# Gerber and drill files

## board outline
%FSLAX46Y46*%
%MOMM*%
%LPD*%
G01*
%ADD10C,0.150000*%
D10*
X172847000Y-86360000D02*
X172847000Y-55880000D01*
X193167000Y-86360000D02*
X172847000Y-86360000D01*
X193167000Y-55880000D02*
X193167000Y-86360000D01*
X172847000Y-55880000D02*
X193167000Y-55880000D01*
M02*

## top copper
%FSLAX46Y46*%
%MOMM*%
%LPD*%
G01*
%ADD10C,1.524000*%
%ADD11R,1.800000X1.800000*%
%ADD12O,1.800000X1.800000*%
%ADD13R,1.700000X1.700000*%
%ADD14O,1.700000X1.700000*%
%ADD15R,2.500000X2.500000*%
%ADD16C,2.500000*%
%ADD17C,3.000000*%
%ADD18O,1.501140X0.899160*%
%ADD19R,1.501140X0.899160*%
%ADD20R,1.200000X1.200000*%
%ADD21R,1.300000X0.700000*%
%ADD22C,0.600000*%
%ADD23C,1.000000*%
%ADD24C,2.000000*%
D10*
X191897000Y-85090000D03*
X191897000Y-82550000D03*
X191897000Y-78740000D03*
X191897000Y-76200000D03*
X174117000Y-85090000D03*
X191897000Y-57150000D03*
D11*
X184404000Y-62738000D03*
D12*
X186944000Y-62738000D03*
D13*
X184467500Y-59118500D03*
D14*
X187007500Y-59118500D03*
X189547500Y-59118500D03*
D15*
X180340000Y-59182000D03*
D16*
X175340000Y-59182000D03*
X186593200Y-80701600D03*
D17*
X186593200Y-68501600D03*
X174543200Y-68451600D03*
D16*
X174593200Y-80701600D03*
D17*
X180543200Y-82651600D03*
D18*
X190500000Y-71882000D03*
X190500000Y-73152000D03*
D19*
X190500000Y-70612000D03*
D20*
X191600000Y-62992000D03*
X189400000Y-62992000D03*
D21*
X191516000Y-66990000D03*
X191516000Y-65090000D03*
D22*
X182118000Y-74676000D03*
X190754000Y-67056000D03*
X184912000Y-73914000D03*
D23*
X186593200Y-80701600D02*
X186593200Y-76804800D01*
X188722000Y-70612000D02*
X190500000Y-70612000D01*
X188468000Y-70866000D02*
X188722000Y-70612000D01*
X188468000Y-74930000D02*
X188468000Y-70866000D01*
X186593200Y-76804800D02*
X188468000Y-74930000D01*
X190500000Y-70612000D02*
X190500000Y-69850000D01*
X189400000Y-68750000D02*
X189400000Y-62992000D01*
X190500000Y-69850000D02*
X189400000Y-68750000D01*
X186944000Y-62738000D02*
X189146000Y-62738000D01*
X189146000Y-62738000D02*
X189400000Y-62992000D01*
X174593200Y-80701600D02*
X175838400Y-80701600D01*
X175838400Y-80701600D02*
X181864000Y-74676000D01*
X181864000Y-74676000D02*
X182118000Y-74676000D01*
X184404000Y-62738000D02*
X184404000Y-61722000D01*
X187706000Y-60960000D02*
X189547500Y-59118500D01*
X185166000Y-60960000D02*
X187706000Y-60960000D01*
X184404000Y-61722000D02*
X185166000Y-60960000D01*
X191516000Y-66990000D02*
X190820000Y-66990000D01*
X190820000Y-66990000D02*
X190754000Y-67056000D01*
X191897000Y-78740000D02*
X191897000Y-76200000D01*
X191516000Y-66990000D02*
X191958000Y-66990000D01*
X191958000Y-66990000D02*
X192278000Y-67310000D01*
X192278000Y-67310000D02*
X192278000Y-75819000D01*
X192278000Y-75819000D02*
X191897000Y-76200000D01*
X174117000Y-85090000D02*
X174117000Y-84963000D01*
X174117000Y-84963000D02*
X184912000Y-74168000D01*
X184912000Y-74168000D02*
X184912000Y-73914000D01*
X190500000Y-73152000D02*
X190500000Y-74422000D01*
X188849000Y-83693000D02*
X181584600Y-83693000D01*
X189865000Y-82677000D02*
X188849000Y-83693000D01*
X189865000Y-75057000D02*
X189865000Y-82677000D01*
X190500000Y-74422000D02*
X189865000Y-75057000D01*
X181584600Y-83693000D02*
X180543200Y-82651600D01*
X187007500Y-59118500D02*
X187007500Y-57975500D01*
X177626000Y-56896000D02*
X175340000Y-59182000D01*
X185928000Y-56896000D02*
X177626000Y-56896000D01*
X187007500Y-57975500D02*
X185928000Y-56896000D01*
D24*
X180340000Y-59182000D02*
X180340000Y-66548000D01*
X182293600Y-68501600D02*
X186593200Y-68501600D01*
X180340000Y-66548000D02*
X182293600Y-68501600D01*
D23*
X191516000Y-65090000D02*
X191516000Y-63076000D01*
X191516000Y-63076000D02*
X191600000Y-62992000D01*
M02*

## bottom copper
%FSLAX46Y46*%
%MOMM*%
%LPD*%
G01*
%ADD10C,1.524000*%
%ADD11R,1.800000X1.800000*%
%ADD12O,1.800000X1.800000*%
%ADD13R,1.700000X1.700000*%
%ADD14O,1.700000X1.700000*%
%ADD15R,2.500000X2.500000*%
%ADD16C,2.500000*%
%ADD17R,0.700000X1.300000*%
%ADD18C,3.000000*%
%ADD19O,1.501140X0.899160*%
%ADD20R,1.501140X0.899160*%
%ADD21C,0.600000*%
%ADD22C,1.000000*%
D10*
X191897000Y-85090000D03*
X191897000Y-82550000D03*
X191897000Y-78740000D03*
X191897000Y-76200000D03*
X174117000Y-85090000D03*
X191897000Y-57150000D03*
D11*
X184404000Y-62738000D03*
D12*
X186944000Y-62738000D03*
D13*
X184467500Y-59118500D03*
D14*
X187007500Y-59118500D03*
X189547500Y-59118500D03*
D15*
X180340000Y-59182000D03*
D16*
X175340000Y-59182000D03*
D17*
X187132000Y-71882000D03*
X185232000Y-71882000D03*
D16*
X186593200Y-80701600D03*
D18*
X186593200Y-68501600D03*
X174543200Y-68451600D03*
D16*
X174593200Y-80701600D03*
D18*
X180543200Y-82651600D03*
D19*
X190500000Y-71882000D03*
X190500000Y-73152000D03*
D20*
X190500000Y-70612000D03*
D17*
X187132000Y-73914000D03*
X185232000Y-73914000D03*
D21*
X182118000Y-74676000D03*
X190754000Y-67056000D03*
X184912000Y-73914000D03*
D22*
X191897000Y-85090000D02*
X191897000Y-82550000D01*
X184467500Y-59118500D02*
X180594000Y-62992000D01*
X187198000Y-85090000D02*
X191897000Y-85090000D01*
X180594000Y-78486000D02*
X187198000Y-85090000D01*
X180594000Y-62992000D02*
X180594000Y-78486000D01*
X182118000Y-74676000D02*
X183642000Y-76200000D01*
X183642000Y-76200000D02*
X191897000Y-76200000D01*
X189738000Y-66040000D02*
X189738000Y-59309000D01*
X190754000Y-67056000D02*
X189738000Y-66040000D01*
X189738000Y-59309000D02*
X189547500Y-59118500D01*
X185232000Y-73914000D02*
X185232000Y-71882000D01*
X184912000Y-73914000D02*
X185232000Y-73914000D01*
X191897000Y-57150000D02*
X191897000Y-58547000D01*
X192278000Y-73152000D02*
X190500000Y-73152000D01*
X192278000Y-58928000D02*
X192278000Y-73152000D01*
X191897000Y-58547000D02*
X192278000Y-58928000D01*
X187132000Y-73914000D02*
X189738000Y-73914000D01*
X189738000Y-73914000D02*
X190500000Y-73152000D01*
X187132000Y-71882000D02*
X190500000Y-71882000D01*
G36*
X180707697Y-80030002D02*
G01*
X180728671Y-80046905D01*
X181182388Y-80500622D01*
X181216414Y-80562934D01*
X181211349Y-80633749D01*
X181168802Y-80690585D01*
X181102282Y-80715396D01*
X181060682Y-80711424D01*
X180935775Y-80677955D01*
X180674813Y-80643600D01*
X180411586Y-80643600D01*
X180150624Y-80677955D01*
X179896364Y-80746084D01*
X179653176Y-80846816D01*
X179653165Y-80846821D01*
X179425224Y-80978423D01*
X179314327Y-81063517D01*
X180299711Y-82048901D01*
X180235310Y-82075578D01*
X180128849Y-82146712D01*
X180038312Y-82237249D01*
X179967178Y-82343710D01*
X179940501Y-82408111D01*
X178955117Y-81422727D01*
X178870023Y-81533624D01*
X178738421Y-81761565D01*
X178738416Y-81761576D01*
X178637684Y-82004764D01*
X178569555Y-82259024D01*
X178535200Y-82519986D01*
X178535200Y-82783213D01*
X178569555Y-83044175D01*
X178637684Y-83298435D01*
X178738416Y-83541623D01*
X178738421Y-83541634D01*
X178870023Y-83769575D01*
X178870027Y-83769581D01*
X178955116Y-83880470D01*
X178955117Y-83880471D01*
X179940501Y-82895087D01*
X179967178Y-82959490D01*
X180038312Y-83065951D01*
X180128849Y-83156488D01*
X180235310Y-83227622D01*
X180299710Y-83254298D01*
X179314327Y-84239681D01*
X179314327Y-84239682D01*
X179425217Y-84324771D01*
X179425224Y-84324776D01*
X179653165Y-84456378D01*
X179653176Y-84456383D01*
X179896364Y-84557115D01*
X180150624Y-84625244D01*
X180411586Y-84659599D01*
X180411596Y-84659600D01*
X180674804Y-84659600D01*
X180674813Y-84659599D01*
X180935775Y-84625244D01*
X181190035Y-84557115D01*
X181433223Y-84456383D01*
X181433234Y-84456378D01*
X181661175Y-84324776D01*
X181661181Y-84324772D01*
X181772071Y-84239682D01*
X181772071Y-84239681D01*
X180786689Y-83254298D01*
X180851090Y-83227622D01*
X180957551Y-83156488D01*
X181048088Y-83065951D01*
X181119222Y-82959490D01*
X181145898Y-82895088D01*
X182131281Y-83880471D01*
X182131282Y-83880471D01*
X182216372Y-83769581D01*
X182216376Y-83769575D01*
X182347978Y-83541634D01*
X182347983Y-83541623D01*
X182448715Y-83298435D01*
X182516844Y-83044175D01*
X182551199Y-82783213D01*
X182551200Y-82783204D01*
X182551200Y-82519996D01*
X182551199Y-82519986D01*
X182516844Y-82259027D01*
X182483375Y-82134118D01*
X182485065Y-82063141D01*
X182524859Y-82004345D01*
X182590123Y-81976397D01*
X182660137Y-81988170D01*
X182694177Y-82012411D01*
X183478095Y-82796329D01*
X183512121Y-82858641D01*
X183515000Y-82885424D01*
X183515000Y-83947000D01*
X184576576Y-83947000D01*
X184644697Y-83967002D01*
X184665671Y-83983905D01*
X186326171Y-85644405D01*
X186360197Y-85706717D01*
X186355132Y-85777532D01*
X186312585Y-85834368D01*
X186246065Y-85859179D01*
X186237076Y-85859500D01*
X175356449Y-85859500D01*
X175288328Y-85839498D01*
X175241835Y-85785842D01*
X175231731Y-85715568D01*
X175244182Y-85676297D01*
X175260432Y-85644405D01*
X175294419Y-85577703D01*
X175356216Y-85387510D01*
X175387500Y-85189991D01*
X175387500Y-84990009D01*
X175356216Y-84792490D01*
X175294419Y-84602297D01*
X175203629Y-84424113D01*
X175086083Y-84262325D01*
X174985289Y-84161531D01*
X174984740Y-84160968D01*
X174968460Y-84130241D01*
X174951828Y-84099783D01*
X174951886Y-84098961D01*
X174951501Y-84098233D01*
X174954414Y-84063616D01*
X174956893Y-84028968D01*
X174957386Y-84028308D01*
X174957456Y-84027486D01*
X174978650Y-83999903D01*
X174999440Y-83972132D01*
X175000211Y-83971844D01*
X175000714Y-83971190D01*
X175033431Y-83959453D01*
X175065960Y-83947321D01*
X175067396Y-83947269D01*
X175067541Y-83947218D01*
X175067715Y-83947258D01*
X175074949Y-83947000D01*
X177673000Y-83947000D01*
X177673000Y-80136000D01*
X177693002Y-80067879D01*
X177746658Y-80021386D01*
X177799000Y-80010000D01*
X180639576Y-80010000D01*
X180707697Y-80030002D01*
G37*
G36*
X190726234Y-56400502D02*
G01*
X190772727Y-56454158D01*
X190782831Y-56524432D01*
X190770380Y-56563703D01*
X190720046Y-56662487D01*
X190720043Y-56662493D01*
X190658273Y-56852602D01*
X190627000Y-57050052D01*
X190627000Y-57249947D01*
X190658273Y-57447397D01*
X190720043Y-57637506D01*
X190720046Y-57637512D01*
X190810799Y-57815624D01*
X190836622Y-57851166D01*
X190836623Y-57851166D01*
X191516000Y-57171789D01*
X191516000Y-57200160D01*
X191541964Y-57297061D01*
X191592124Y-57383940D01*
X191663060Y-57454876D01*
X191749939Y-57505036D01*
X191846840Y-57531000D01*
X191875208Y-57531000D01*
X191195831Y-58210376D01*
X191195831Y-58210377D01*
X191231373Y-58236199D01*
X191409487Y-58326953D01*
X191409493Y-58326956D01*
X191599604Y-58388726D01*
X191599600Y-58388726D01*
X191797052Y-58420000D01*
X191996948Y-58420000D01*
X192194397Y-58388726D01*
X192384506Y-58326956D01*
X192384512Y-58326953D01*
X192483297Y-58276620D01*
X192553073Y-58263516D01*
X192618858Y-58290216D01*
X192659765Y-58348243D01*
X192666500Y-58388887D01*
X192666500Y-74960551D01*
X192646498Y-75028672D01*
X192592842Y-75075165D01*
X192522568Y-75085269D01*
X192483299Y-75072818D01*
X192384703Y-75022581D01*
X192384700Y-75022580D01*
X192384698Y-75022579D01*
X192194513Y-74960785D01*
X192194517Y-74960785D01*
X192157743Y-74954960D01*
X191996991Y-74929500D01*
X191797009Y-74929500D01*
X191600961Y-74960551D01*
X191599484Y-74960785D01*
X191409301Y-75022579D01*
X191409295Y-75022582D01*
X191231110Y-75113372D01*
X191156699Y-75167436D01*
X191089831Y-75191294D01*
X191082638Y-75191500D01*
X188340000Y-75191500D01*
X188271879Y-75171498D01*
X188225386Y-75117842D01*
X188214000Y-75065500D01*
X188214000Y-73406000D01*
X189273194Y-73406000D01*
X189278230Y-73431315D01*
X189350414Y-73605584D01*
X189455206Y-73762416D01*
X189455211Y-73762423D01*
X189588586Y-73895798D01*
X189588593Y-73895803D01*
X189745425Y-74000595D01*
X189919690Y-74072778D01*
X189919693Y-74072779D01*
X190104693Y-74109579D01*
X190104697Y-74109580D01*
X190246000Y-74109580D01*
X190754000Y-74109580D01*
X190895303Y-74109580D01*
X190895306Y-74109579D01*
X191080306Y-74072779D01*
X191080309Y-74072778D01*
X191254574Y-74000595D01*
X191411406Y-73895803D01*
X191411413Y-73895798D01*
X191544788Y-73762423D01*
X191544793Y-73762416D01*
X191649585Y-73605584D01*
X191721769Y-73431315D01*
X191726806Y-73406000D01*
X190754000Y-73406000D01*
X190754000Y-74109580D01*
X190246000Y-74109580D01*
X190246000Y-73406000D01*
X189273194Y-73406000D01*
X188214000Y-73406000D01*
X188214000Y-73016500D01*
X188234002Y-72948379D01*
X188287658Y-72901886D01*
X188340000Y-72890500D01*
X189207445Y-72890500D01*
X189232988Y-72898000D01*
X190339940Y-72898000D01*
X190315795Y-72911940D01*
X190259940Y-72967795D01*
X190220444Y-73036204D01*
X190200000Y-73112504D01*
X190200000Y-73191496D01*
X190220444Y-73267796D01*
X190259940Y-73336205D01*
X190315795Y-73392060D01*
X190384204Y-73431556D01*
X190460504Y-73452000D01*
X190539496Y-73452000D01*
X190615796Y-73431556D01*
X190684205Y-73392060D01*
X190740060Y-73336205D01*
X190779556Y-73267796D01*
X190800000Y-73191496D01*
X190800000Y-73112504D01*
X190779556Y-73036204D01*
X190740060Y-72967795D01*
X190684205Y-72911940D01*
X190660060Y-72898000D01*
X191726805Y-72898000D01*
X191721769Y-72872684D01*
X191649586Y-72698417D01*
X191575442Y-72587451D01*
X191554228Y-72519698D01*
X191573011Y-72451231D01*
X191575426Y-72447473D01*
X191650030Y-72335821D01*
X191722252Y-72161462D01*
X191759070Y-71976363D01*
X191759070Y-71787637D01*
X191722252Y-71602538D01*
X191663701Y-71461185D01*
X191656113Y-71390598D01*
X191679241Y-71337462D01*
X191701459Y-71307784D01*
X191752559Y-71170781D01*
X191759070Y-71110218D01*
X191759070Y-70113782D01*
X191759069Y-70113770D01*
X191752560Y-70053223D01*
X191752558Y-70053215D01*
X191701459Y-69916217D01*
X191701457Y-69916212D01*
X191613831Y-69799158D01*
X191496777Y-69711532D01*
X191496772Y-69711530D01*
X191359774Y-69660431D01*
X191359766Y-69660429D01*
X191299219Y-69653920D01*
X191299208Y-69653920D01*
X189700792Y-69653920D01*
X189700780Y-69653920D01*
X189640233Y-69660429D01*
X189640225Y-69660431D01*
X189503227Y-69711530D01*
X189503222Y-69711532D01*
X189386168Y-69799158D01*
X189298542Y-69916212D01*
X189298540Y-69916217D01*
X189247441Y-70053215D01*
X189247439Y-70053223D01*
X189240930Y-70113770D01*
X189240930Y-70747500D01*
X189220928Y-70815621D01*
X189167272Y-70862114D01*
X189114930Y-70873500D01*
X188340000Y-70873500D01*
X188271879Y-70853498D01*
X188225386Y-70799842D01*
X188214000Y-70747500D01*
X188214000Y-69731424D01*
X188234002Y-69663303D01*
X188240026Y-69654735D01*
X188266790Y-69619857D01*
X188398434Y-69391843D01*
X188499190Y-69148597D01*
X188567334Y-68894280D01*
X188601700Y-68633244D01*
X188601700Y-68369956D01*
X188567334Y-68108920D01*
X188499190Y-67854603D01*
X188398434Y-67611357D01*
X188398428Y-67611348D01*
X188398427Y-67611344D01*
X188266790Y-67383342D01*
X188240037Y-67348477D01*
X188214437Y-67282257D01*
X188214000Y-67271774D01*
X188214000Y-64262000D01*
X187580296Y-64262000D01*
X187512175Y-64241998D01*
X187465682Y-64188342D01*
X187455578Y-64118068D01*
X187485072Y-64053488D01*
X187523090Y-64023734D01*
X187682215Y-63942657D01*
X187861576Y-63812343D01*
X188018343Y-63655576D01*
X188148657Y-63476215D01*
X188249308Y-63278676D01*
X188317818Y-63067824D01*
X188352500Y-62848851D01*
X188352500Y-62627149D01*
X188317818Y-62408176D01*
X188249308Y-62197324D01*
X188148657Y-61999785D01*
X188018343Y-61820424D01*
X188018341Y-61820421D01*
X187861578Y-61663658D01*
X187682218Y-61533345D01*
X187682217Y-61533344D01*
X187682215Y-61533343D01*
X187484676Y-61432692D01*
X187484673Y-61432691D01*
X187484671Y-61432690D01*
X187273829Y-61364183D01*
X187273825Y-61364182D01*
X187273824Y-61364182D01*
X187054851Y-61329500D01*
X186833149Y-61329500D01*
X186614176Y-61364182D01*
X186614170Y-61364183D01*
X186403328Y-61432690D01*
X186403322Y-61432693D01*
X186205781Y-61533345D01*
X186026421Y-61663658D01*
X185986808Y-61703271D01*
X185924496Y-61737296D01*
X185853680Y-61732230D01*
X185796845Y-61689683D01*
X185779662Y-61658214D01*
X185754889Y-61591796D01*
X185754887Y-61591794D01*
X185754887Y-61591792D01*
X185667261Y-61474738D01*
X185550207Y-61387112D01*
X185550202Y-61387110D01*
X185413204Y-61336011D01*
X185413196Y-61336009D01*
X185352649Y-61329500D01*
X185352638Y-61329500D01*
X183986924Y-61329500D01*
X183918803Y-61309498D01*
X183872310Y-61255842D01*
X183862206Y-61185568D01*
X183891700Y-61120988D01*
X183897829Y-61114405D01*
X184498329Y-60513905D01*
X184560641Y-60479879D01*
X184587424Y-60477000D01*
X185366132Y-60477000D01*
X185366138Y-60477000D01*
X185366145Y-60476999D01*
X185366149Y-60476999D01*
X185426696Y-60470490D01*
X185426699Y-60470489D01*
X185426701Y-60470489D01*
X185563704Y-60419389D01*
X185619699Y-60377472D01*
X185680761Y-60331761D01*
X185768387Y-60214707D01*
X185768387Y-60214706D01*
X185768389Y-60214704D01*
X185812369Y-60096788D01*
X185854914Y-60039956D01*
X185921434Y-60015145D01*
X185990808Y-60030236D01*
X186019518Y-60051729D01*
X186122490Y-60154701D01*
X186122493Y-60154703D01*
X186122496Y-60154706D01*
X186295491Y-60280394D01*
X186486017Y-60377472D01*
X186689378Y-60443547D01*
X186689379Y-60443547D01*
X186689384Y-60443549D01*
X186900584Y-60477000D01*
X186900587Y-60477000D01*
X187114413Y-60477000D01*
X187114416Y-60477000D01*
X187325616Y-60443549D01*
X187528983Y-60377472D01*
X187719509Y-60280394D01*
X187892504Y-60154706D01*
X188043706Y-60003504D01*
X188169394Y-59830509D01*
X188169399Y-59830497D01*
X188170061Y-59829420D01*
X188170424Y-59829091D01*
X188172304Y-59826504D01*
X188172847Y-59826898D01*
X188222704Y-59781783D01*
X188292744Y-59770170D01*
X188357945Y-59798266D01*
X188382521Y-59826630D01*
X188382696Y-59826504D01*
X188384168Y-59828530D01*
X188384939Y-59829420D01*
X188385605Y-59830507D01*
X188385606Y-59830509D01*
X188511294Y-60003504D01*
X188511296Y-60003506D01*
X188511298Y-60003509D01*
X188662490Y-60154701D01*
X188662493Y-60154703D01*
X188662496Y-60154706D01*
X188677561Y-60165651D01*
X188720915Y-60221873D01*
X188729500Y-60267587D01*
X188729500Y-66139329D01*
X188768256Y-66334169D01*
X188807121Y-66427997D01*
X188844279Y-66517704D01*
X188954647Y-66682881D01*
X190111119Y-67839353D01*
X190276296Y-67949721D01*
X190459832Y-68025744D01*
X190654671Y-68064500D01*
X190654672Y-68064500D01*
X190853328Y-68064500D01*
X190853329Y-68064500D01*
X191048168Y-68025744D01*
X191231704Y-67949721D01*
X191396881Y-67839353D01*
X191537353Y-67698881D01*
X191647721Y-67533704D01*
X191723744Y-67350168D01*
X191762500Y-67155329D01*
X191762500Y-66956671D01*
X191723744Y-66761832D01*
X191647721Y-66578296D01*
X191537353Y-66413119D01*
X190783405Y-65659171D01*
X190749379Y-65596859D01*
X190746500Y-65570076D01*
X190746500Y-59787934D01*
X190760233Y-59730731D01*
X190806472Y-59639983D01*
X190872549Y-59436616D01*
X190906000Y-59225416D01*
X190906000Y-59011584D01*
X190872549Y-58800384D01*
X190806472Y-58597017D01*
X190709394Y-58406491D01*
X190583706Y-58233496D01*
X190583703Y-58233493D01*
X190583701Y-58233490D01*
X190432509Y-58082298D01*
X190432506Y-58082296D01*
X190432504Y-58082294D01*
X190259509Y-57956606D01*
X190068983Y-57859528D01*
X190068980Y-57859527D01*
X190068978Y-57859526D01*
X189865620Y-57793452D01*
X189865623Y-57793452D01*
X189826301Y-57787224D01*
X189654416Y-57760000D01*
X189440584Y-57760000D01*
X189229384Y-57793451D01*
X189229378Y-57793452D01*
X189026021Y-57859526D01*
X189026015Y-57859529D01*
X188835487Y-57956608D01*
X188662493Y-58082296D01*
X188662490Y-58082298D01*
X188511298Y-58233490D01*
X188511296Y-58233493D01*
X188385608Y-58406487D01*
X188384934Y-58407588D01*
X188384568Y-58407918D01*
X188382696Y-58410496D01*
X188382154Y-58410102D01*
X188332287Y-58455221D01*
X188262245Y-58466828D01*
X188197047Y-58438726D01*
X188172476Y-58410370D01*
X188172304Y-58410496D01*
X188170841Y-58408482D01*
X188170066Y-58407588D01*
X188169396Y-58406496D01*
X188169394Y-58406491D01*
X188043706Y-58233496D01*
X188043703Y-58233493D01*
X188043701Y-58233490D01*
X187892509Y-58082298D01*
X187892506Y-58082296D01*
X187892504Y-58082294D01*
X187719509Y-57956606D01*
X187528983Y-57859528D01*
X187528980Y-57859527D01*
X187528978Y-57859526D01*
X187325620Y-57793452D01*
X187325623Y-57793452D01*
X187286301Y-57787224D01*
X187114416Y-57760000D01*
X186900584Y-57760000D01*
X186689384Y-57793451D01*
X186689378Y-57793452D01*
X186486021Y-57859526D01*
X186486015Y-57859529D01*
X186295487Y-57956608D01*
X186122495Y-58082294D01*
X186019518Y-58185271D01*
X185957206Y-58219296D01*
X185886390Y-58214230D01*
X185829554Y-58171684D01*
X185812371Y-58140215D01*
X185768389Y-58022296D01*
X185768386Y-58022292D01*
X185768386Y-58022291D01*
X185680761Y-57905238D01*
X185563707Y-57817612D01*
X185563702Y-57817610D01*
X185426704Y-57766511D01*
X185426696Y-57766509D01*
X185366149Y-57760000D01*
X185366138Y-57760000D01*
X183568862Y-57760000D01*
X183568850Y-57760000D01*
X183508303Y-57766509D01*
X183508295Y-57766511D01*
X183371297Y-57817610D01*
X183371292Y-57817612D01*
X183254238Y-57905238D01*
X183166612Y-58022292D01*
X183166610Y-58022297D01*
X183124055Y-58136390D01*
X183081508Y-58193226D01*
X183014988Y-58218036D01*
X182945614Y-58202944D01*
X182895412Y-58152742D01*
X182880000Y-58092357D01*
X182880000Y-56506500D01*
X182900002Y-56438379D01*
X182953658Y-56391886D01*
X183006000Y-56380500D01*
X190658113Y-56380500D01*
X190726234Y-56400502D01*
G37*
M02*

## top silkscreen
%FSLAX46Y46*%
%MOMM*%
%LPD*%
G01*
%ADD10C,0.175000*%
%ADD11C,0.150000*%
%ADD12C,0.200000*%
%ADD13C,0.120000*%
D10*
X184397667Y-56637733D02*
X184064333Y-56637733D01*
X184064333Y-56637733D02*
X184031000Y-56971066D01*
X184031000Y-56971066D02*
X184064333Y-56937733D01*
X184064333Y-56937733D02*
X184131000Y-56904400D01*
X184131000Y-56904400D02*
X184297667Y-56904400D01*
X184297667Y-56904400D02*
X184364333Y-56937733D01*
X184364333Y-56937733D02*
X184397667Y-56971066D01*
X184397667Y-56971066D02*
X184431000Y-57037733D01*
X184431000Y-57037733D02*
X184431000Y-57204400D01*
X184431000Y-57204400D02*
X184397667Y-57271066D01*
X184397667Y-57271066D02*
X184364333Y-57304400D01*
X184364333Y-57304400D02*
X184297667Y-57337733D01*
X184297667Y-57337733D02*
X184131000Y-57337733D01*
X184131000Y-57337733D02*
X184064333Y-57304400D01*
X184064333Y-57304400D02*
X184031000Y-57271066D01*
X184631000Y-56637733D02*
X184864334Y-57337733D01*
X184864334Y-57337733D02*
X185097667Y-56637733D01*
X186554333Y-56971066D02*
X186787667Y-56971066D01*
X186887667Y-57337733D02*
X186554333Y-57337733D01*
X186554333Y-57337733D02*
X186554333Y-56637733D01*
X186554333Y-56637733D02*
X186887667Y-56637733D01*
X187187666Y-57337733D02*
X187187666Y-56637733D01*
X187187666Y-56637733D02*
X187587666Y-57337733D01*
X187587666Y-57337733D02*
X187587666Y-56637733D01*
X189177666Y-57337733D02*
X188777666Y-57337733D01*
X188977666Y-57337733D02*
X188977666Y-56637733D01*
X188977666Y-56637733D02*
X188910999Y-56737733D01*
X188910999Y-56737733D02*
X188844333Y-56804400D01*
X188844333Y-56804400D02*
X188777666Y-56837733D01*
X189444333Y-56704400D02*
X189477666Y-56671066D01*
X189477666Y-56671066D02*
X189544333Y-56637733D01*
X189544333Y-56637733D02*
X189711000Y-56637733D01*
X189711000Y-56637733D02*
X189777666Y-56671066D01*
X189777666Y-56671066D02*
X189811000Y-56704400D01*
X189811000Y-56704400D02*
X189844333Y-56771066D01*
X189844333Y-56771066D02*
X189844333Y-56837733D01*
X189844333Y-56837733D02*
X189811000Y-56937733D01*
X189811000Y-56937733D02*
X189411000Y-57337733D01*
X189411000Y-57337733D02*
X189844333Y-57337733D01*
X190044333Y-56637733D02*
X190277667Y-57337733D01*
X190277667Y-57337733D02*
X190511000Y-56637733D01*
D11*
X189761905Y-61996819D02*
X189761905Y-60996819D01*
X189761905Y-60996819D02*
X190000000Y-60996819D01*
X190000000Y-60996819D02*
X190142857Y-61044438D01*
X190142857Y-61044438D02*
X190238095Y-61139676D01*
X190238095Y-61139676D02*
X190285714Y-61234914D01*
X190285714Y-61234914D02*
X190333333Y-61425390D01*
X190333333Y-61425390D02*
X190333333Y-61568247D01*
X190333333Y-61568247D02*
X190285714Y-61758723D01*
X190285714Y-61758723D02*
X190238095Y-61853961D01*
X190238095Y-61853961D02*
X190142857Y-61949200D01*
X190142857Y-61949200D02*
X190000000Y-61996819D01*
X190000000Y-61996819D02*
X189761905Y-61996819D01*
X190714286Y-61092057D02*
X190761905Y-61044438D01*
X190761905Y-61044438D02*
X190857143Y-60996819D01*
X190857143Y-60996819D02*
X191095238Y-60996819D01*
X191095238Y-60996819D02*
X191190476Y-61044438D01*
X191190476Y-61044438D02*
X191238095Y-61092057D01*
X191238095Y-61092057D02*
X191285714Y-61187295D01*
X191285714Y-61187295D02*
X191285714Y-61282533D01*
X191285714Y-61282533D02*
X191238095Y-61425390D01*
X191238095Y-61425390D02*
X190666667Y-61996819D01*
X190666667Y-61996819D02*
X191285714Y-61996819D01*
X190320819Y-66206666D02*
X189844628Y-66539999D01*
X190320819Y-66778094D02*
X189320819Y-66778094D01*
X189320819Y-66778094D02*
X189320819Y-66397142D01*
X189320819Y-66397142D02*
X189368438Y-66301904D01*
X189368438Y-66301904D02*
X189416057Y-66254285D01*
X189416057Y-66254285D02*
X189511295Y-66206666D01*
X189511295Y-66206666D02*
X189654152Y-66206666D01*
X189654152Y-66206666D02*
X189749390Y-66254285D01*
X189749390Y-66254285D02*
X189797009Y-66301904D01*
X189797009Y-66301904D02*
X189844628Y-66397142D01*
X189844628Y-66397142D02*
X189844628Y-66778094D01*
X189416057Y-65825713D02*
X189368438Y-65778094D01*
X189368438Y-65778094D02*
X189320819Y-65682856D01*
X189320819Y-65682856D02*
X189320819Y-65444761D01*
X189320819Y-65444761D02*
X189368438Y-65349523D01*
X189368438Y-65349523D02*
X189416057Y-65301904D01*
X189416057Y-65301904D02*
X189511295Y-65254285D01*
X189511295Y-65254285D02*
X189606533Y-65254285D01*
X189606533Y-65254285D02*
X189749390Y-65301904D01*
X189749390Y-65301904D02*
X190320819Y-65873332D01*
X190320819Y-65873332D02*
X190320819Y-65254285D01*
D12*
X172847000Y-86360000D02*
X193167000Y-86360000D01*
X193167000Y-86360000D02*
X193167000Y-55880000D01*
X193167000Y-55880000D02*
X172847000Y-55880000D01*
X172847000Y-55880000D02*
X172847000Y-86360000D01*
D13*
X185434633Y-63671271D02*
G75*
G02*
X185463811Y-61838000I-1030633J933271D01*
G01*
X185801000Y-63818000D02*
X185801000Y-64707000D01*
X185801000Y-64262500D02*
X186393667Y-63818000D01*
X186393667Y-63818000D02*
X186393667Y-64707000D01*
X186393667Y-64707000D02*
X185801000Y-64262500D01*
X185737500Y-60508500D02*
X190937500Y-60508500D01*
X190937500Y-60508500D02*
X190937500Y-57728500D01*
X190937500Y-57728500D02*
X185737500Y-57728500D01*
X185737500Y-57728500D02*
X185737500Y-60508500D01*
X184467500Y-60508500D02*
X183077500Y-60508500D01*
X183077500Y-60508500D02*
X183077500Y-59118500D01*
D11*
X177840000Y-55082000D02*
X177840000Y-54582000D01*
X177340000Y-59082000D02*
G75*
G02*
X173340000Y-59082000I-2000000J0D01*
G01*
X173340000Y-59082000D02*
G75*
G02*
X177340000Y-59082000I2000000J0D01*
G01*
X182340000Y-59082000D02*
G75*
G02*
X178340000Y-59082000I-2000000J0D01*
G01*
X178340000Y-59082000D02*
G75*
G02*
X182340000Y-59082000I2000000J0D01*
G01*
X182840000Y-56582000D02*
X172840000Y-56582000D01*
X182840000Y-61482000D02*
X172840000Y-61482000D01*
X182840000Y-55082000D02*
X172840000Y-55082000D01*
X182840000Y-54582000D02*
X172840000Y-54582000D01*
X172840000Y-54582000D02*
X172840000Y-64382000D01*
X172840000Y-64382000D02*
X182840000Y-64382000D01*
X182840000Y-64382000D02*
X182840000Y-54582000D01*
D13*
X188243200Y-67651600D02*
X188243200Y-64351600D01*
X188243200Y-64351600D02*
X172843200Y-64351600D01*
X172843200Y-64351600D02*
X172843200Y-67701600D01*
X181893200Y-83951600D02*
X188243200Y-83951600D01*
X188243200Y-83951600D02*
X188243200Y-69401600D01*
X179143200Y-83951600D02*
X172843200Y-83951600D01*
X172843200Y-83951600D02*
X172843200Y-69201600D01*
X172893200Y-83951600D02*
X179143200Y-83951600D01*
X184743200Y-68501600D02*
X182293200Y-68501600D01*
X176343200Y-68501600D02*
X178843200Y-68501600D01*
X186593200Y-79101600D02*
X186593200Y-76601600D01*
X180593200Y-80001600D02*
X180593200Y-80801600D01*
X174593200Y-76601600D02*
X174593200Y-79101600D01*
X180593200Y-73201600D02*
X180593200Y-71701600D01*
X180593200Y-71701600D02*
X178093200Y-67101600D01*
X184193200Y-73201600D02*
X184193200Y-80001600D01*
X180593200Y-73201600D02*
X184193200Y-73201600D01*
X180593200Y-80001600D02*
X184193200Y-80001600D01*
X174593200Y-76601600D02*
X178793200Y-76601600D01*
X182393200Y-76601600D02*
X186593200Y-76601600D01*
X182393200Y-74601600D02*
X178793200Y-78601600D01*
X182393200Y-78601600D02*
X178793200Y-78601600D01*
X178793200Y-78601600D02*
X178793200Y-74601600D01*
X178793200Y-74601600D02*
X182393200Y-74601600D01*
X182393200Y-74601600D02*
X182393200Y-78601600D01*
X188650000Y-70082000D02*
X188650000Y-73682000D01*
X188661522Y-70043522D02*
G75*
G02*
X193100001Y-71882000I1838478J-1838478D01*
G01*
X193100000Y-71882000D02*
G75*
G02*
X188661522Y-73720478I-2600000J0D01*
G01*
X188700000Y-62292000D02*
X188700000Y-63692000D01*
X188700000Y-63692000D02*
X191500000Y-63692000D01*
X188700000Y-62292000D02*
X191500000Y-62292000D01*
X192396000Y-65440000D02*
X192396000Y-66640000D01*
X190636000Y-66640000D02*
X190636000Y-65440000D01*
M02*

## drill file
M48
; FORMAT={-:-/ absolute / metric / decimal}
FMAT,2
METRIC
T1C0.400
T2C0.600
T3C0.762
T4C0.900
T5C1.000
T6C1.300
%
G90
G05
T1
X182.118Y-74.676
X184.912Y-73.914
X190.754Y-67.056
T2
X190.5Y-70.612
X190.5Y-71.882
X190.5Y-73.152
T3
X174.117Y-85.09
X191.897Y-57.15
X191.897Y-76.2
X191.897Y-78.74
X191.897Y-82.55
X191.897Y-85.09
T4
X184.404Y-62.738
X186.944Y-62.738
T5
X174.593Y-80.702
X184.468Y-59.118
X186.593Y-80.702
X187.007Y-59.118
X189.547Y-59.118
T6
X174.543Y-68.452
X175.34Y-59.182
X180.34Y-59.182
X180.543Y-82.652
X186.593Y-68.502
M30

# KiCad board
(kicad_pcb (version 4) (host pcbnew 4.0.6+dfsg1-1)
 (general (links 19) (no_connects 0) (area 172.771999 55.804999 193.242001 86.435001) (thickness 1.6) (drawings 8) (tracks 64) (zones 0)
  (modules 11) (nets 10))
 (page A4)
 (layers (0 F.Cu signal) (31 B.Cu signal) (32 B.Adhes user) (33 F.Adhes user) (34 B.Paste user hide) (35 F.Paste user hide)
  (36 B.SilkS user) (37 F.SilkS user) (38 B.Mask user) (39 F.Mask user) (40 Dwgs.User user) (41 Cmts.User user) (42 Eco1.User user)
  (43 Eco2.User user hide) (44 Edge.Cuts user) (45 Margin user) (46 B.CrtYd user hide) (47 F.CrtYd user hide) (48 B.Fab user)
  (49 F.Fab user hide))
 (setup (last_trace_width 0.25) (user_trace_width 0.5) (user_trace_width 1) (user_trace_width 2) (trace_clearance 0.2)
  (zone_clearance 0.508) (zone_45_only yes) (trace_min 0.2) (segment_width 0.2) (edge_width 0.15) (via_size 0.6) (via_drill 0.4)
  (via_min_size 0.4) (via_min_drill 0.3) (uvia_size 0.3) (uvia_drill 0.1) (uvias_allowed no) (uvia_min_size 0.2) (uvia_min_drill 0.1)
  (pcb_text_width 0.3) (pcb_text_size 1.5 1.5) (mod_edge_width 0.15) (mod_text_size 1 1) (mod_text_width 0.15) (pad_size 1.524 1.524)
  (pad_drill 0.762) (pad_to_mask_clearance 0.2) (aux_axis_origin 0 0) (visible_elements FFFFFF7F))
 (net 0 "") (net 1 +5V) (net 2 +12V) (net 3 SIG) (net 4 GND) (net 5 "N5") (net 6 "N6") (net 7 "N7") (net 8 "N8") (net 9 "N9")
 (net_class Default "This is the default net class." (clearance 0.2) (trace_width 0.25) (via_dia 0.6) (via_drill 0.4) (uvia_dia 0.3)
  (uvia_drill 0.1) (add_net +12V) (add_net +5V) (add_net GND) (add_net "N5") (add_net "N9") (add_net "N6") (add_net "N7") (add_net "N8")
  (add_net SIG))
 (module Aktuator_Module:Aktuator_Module (layer F.Cu) (at 172.847 86.36)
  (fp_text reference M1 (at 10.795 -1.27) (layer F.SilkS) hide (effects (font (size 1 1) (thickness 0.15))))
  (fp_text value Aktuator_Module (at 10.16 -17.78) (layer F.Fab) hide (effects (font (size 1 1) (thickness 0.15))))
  (fp_line (start 0 0) (end 20.32 0) (layer F.SilkS) (width 0.2))
  (fp_line (start 20.32 0) (end 20.32 -30.48) (layer F.SilkS) (width 0.2))
  (fp_line (start 20.32 -30.48) (end 0 -30.48) (layer F.SilkS) (width 0.2))
  (fp_line (start 0 -30.48) (end 0 0) (layer F.SilkS) (width 0.2))
  (pad 1 thru_hole circle (at 19.05 -1.27) (size 1.524 1.524) (drill 0.762) (layers *.Cu *.Mask) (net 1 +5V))
  (pad 1 thru_hole circle (at 19.05 -3.81) (size 1.524 1.524) (drill 0.762) (layers *.Cu *.Mask) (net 1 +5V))
  (pad 2 thru_hole circle (at 19.05 -7.62) (size 1.524 1.524) (drill 0.762) (layers *.Cu *.Mask) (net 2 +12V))
  (pad 2 thru_hole circle (at 19.05 -10.16) (size 1.524 1.524) (drill 0.762) (layers *.Cu *.Mask) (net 2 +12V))
  (pad 3 thru_hole circle (at 1.27 -1.27) (size 1.524 1.524) (drill 0.762) (layers *.Cu *.Mask) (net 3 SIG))
  (pad 4 thru_hole circle (at 19.05 -29.21) (size 1.524 1.524) (drill 0.762) (layers *.Cu *.Mask) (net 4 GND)))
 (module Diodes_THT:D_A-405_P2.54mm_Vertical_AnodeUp (layer F.Cu) (at 184.404 62.738)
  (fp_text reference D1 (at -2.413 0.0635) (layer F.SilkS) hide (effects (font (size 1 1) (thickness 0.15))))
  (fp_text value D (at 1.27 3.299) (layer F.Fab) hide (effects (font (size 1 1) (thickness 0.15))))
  (fp_arc (start 0 0) (end 1.059811 -0.9) (angle -277.5) (layer F.SilkS) (width 0.12))
  (fp_line (start 1.397 1.08) (end 1.397 1.969) (layer F.SilkS) (width 0.12))
  (fp_line (start 1.397 1.5245) (end 1.989667 1.08) (layer F.SilkS) (width 0.12))
  (fp_line (start 1.989667 1.08) (end 1.989667 1.969) (layer F.SilkS) (width 0.12))
  (fp_line (start 1.989667 1.969) (end 1.397 1.5245) (layer F.SilkS) (width 0.12))
  (pad 1 thru_hole rect (at 0 0) (size 1.8 1.8) (drill 0.9) (layers *.Cu *.Mask) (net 2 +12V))
  (pad 2 thru_hole oval (at 2.54 0) (size 1.8 1.8) (drill 0.9) (layers *.Cu *.Mask) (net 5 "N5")))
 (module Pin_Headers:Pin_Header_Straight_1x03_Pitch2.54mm (layer F.Cu) (at 184.4675 59.1185 90)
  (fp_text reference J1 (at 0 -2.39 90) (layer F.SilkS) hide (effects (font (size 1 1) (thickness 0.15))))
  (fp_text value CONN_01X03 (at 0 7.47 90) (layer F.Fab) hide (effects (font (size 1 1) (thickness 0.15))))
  (fp_line (start -1.39 1.27) (end -1.39 6.47) (layer F.SilkS) (width 0.12))
  (fp_line (start -1.39 6.47) (end 1.39 6.47) (layer F.SilkS) (width 0.12))
  (fp_line (start 1.39 6.47) (end 1.39 1.27) (layer F.SilkS) (width 0.12))
  (fp_line (start 1.39 1.27) (end -1.39 1.27) (layer F.SilkS) (width 0.12))
  (fp_line (start -1.39 0) (end -1.39 -1.39) (layer F.SilkS) (width 0.12))
  (fp_line (start -1.39 -1.39) (end 0 -1.39) (layer F.SilkS) (width 0.12))
  (pad 1 thru_hole rect (at 0 0 90) (size 1.7 1.7) (drill 1) (layers *.Cu *.Mask) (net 1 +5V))
  (pad 2 thru_hole oval (at 0 2.54 90) (size 1.7 1.7) (drill 1) (layers *.Cu *.Mask) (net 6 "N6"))
  (pad 3 thru_hole oval (at 0 5.08 90) (size 1.7 1.7) (drill 1) (layers *.Cu *.Mask) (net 2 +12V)))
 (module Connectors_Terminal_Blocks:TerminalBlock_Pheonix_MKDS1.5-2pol (layer F.Cu) (at 180.34 59.182 180)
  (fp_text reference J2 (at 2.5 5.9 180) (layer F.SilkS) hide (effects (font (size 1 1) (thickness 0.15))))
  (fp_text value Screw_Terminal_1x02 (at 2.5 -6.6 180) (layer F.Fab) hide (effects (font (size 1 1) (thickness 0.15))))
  (fp_line (start 2.5 4.1) (end 2.5 4.6) (layer F.SilkS) (width 0.15))
  (fp_circle (center 5 0.1) (end 3 0.1) (layer F.SilkS) (width 0.15))
  (fp_circle (center 0 0.1) (end 2 0.1) (layer F.SilkS) (width 0.15))
  (fp_line (start -2.5 2.6) (end 7.5 2.6) (layer F.SilkS) (width 0.15))
  (fp_line (start -2.5 -2.3) (end 7.5 -2.3) (layer F.SilkS) (width 0.15))
  (fp_line (start -2.5 4.1) (end 7.5 4.1) (layer F.SilkS) (width 0.15))
  (fp_line (start -2.5 4.6) (end 7.5 4.6) (layer F.SilkS) (width 0.15))
  (fp_line (start 7.5 4.6) (end 7.5 -5.2) (layer F.SilkS) (width 0.15))
  (fp_line (start 7.5 -5.2) (end -2.5 -5.2) (layer F.SilkS) (width 0.15))
  (fp_line (start -2.5 -5.2) (end -2.5 4.6) (layer F.SilkS) (width 0.15))
  (pad 1 thru_hole rect (at 0 0 180) (size 2.5 2.5) (drill 1.3) (layers *.Cu *.Mask) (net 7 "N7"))
  (pad 2 thru_hole circle (at 5 0 180) (size 2.5 2.5) (drill 1.3) (layers *.Cu *.Mask) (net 6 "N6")))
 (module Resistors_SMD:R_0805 (layer B.Cu) (at 186.182 71.882 180)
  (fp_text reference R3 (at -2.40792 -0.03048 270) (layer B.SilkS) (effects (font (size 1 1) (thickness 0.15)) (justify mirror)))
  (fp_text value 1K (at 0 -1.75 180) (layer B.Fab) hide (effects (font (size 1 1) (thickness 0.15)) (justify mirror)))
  (pad 1 smd rect (at -0.95 0 180) (size 0.7 1.3) (layers B.Cu B.Paste B.Mask) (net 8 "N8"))
  (pad 2 smd rect (at 0.95 0 180) (size 0.7 1.3) (layers B.Cu B.Paste B.Mask) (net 3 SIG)))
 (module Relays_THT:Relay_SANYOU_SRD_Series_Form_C (layer F.Cu) (at 180.5432 82.6516 90)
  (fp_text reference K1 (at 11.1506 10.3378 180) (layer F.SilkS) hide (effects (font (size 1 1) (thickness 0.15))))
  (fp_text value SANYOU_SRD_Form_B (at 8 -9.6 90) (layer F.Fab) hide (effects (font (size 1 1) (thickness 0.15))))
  (fp_line (start 15 7.7) (end 18.3 7.7) (layer F.SilkS) (width 0.12))
  (fp_line (start 18.3 7.7) (end 18.3 -7.7) (layer F.SilkS) (width 0.12))
  (fp_line (start 18.3 -7.7) (end 14.95 -7.7) (layer F.SilkS) (width 0.12))
  (fp_line (start -1.3 1.35) (end -1.3 7.7) (layer F.SilkS) (width 0.12))
  (fp_line (start -1.3 7.7) (end 13.25 7.7) (layer F.SilkS) (width 0.12))
  (fp_line (start -1.3 -1.4) (end -1.3 -7.7) (layer F.SilkS) (width 0.12))
  (fp_line (start -1.3 -7.7) (end 13.45 -7.7) (layer F.SilkS) (width 0.12))
  (fp_line (start -1.3 -7.65) (end -1.3 -1.4) (layer F.SilkS) (width 0.12))
  (fp_line (start 14.15 4.2) (end 14.15 1.75) (layer F.SilkS) (width 0.12))
  (fp_line (start 14.15 -4.2) (end 14.15 -1.7) (layer F.SilkS) (width 0.12))
  (fp_line (start 3.55 6.05) (end 6.05 6.05) (layer F.SilkS) (width 0.12))
  (fp_line (start 2.65 0.05) (end 1.85 0.05) (layer F.SilkS) (width 0.12))
  (fp_line (start 6.05 -5.95) (end 3.55 -5.95) (layer F.SilkS) (width 0.12))
  (fp_line (start 9.45 0.05) (end 10.95 0.05) (layer F.SilkS) (width 0.12))
  (fp_line (start 10.95 0.05) (end 15.55 -2.45) (layer F.SilkS) (width 0.12))
  (fp_line (start 9.45 3.65) (end 2.65 3.65) (layer F.SilkS) (width 0.12))
  (fp_line (start 9.45 0.05) (end 9.45 3.65) (layer F.SilkS) (width 0.12))
  (fp_line (start 2.65 0.05) (end 2.65 3.65) (layer F.SilkS) (width 0.12))
  (fp_line (start 6.05 -5.95) (end 6.05 -1.75) (layer F.SilkS) (width 0.12))
  (fp_line (start 6.05 1.85) (end 6.05 6.05) (layer F.SilkS) (width 0.12))
  (fp_line (start 8.05 1.85) (end 4.05 -1.75) (layer F.SilkS) (width 0.12))
  (fp_line (start 4.05 1.85) (end 4.05 -1.75) (layer F.SilkS) (width 0.12))
  (fp_line (start 4.05 -1.75) (end 8.05 -1.75) (layer F.SilkS) (width 0.12))
  (fp_line (start 8.05 -1.75) (end 8.05 1.85) (layer F.SilkS) (width 0.12))
  (fp_line (start 8.05 1.85) (end 4.05 1.85) (layer F.SilkS) (width 0.12))
  (pad 2 thru_hole circle (at 1.95 6.05 180) (size 2.5 2.5) (drill 1) (layers *.Cu *.Mask) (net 5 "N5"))
  (pad 3 thru_hole circle (at 14.15 6.05 180) (size 3 3) (drill 1.3) (layers *.Cu *.Mask) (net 7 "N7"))
  (pad 4 thru_hole circle (at 14.2 -6 180) (size 3 3) (drill 1.3) (layers *.Cu *.Mask))
  (pad 5 thru_hole circle (at 1.95 -5.95 180) (size 2.5 2.5) (drill 1) (layers *.Cu *.Mask) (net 2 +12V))
  (pad 1 thru_hole circle (at 0 0 180) (size 3 3) (drill 1.3) (layers *.Cu *.Mask) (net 4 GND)))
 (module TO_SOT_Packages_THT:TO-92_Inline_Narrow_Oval (layer F.Cu) (at 190.5 70.612 270)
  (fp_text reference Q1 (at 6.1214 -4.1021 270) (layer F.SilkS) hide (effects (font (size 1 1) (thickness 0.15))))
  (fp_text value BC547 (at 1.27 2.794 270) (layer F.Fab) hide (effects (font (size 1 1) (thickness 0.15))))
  (fp_line (start -0.53 1.85) (end 3.07 1.85) (layer F.SilkS) (width 0.12))
  (fp_arc (start 1.27 0) (end 1.27 -2.6) (angle -135) (layer F.SilkS) (width 0.12))
  (fp_arc (start 1.27 0) (end 1.27 -2.6) (angle 135) (layer F.SilkS) (width 0.12))
  (pad 2 thru_hole oval (at 1.27 0 90) (size 0.89916 1.50114) (drill 0.6) (layers *.Cu *.Mask) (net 8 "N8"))
  (pad 3 thru_hole oval (at 2.54 0 90) (size 0.89916 1.50114) (drill 0.6) (layers *.Cu *.Mask) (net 4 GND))
  (pad 1 thru_hole rect (at 0 0 90) (size 0.89916 1.50114) (drill 0.6) (layers *.Cu *.Mask) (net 5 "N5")))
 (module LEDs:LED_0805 (layer F.Cu) (at 190.5 62.992)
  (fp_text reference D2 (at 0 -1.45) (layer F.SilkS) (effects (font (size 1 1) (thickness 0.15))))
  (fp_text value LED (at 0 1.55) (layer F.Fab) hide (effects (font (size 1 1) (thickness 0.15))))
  (fp_line (start -1.8 -0.7) (end -1.8 0.7) (layer F.SilkS) (width 0.12))
  (fp_line (start -1.8 0.7) (end 1 0.7) (layer F.SilkS) (width 0.12))
  (fp_line (start -1.8 -0.7) (end 1 -0.7) (layer F.SilkS) (width 0.12))
  (pad 2 smd rect (at 1.1 0 180) (size 1.2 1.2) (layers F.Cu F.Paste F.Mask) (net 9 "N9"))
  (pad 1 smd rect (at -1.1 0 180) (size 1.2 1.2) (layers F.Cu F.Paste F.Mask) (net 5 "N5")))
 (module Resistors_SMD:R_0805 (layer B.Cu) (at 186.182 73.914 180)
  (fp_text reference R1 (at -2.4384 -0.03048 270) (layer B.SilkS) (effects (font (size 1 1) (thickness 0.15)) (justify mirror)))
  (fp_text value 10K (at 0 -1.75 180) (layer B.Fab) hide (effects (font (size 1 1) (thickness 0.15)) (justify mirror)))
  (pad 1 smd rect (at -0.95 0 180) (size 0.7 1.3) (layers B.Cu B.Paste B.Mask) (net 4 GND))
  (pad 2 smd rect (at 0.95 0 180) (size 0.7 1.3) (layers B.Cu B.Paste B.Mask) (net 3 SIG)))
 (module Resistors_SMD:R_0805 (layer F.Cu) (at 191.516 66.04 90)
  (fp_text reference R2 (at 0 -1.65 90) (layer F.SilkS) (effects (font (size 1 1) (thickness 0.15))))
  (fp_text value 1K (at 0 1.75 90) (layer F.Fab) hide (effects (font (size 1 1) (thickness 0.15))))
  (fp_line (start 0.6 0.88) (end -0.6 0.88) (layer F.SilkS) (width 0.12))
  (fp_line (start -0.6 -0.88) (end 0.6 -0.88) (layer F.SilkS) (width 0.12))
  (pad 1 smd rect (at -0.95 0 90) (size 0.7 1.3) (layers F.Cu F.Paste F.Mask) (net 2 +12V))
  (pad 2 smd rect (at 0.95 0 90) (size 0.7 1.3) (layers F.Cu F.Paste F.Mask) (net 9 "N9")))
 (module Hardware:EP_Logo (layer B.Cu) (at 179.451 74.676 180)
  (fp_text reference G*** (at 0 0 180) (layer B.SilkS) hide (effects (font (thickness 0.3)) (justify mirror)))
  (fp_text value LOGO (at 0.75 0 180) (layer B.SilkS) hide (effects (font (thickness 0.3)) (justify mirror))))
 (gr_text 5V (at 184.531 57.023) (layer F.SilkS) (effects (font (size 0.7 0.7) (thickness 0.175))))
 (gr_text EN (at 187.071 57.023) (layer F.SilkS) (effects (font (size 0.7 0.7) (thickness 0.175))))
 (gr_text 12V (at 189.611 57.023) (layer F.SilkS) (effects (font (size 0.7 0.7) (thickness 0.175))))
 (gr_line (start 172.847 86.36) (end 172.847 55.88) (angle 90) (layer Edge.Cuts) (width 0.15))
 (gr_line (start 193.167 86.36) (end 172.847 86.36) (angle 90) (layer Edge.Cuts) (width 0.15))
 (gr_line (start 193.167 55.88) (end 193.167 86.36) (angle 90) (layer Edge.Cuts) (width 0.15))
 (gr_line (start 172.847 55.88) (end 193.167 55.88) (angle 90) (layer Edge.Cuts) (width 0.15))
 (segment (start 186.5932 80.7016) (end 186.5932 76.8048) (width 1) (layer F.Cu) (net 5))
 (segment (start 188.722 70.612) (end 190.5 70.612) (width 1) (layer F.Cu) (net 5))
 (segment (start 188.468 70.866) (end 188.722 70.612) (width 1) (layer F.Cu) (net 5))
 (segment (start 188.468 74.93) (end 188.468 70.866) (width 1) (layer F.Cu) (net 5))
 (segment (start 186.5932 76.8048) (end 188.468 74.93) (width 1) (layer F.Cu) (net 5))
 (segment (start 190.5 70.612) (end 190.5 69.85) (width 1) (layer F.Cu) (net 5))
 (segment (start 189.4 68.75) (end 189.4 62.992) (width 1) (layer F.Cu) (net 5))
 (segment (start 190.5 69.85) (end 189.4 68.75) (width 1) (layer F.Cu) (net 5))
 (segment (start 186.944 62.738) (end 189.146 62.738) (width 1) (layer F.Cu) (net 5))
 (segment (start 189.146 62.738) (end 189.4 62.992) (width 1) (layer F.Cu) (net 5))
 (segment (start 191.897 85.09) (end 191.897 82.55) (width 1) (layer B.Cu) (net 1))
 (segment (start 184.4675 59.1185) (end 180.594 62.992) (width 1) (layer B.Cu) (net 1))
 (segment (start 187.198 85.09) (end 191.897 85.09) (width 1) (layer B.Cu) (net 1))
 (segment (start 180.594 78.486) (end 187.198 85.09) (width 1) (layer B.Cu) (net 1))
 (segment (start 180.594 62.992) (end 180.594 78.486) (width 1) (layer B.Cu) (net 1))
 (segment (start 174.5932 80.7016) (end 175.8384 80.7016) (width 1) (layer F.Cu) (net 2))
 (segment (start 175.8384 80.7016) (end 181.864 74.676) (width 1) (layer F.Cu) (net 2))
 (segment (start 181.864 74.676) (end 182.118 74.676) (width 1) (layer F.Cu) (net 2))
 (via (at 182.118 74.676) (size 0.6) (drill 0.4) (layers F.Cu B.Cu) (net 2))
 (segment (start 182.118 74.676) (end 183.642 76.2) (width 1) (layer B.Cu) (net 2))
 (segment (start 183.642 76.2) (end 191.897 76.2) (width 1) (layer B.Cu) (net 2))
 (segment (start 184.404 62.738) (end 184.404 61.722) (width 1) (layer F.Cu) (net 2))
 (segment (start 187.706 60.96) (end 189.5475 59.1185) (width 1) (layer F.Cu) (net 2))
 (segment (start 185.166 60.96) (end 187.706 60.96) (width 1) (layer F.Cu) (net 2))
 (segment (start 184.404 61.722) (end 185.166 60.96) (width 1) (layer F.Cu) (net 2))
 (segment (start 191.516 66.99) (end 190.82 66.99) (width 1) (layer F.Cu) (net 2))
 (segment (start 189.738 66.04) (end 189.738 59.309) (width 1) (layer B.Cu) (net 2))
 (segment (start 190.754 67.056) (end 189.738 66.04) (width 1) (layer B.Cu) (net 2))
 (via (at 190.754 67.056) (size 0.6) (drill 0.4) (layers F.Cu B.Cu) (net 2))
 (segment (start 190.82 66.99) (end 190.754 67.056) (width 1) (layer F.Cu) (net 2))
 (segment (start 189.738 59.309) (end 189.5475 59.1185) (width 1) (layer B.Cu) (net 2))
 (segment (start 191.897 78.74) (end 191.897 76.2) (width 1) (layer F.Cu) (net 2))
 (segment (start 191.516 66.99) (end 191.958 66.99) (width 1) (layer F.Cu) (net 2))
 (segment (start 191.958 66.99) (end 192.278 67.31) (width 1) (layer F.Cu) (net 2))
 (segment (start 192.278 67.31) (end 192.278 75.819) (width 1) (layer F.Cu) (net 2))
 (segment (start 192.278 75.819) (end 191.897 76.2) (width 1) (layer F.Cu) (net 2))
 (segment (start 185.232 73.914) (end 185.232 71.882) (width 1) (layer B.Cu) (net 3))
 (segment (start 174.117 85.09) (end 174.117 84.963) (width 1) (layer F.Cu) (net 3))
 (segment (start 174.117 84.963) (end 184.912 74.168) (width 1) (layer F.Cu) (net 3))
 (segment (start 184.912 74.168) (end 184.912 73.914) (width 1) (layer F.Cu) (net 3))
 (via (at 184.912 73.914) (size 0.6) (drill 0.4) (layers F.Cu B.Cu) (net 3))
 (segment (start 184.912 73.914) (end 185.232 73.914) (width 1) (layer B.Cu) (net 3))
 (segment (start 190.5 73.152) (end 190.5 74.422) (width 1) (layer F.Cu) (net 4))
 (segment (start 188.849 83.693) (end 181.5846 83.693) (width 1) (layer F.Cu) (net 4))
 (segment (start 189.865 82.677) (end 188.849 83.693) (width 1) (layer F.Cu) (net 4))
 (segment (start 189.865 75.057) (end 189.865 82.677) (width 1) (layer F.Cu) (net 4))
 (segment (start 190.5 74.422) (end 189.865 75.057) (width 1) (layer F.Cu) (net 4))
 (segment (start 181.5846 83.693) (end 180.5432 82.6516) (width 1) (layer F.Cu) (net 4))
 (segment (start 191.897 57.15) (end 191.897 58.547) (width 1) (layer B.Cu) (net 4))
 (segment (start 192.278 73.152) (end 190.5 73.152) (width 1) (layer B.Cu) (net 4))
 (segment (start 192.278 58.928) (end 192.278 73.152) (width 1) (layer B.Cu) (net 4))
 (segment (start 191.897 58.547) (end 192.278 58.928) (width 1) (layer B.Cu) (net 4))
 (segment (start 187.132 73.914) (end 189.738 73.914) (width 1) (layer B.Cu) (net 4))
 (segment (start 189.738 73.914) (end 190.5 73.152) (width 1) (layer B.Cu) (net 4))
 (segment (start 187.132 71.882) (end 190.5 71.882) (width 1) (layer B.Cu) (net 8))
 (segment (start 187.0075 59.1185) (end 187.0075 57.9755) (width 1) (layer F.Cu) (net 6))
 (segment (start 177.626 56.896) (end 175.34 59.182) (width 1) (layer F.Cu) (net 6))
 (segment (start 185.928 56.896) (end 177.626 56.896) (width 1) (layer F.Cu) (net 6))
 (segment (start 187.0075 57.9755) (end 185.928 56.896) (width 1) (layer F.Cu) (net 6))
 (segment (start 180.34 59.182) (end 180.34 66.548) (width 2) (layer F.Cu) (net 7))
 (segment (start 182.2936 68.5016) (end 186.5932 68.5016) (width 2) (layer F.Cu) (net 7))
 (segment (start 180.34 66.548) (end 182.2936 68.5016) (width 2) (layer F.Cu) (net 7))
 (segment (start 191.516 65.09) (end 191.516 63.076) (width 1) (layer F.Cu) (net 9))
 (segment (start 191.516 63.076) (end 191.6 62.992) (width 1) (layer F.Cu) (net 9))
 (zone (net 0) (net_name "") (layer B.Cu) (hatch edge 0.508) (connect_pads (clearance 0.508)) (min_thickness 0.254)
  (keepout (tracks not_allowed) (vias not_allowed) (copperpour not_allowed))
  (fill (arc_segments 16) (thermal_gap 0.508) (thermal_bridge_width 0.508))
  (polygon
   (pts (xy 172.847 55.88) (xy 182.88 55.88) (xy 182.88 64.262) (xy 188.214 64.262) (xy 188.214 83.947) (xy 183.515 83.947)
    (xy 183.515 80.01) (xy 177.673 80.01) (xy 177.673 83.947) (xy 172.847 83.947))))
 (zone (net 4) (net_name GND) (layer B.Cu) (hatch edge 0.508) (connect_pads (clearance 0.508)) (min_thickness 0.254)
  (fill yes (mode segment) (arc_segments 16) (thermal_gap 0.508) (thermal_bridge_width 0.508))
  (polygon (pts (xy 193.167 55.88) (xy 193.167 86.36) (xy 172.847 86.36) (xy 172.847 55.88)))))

